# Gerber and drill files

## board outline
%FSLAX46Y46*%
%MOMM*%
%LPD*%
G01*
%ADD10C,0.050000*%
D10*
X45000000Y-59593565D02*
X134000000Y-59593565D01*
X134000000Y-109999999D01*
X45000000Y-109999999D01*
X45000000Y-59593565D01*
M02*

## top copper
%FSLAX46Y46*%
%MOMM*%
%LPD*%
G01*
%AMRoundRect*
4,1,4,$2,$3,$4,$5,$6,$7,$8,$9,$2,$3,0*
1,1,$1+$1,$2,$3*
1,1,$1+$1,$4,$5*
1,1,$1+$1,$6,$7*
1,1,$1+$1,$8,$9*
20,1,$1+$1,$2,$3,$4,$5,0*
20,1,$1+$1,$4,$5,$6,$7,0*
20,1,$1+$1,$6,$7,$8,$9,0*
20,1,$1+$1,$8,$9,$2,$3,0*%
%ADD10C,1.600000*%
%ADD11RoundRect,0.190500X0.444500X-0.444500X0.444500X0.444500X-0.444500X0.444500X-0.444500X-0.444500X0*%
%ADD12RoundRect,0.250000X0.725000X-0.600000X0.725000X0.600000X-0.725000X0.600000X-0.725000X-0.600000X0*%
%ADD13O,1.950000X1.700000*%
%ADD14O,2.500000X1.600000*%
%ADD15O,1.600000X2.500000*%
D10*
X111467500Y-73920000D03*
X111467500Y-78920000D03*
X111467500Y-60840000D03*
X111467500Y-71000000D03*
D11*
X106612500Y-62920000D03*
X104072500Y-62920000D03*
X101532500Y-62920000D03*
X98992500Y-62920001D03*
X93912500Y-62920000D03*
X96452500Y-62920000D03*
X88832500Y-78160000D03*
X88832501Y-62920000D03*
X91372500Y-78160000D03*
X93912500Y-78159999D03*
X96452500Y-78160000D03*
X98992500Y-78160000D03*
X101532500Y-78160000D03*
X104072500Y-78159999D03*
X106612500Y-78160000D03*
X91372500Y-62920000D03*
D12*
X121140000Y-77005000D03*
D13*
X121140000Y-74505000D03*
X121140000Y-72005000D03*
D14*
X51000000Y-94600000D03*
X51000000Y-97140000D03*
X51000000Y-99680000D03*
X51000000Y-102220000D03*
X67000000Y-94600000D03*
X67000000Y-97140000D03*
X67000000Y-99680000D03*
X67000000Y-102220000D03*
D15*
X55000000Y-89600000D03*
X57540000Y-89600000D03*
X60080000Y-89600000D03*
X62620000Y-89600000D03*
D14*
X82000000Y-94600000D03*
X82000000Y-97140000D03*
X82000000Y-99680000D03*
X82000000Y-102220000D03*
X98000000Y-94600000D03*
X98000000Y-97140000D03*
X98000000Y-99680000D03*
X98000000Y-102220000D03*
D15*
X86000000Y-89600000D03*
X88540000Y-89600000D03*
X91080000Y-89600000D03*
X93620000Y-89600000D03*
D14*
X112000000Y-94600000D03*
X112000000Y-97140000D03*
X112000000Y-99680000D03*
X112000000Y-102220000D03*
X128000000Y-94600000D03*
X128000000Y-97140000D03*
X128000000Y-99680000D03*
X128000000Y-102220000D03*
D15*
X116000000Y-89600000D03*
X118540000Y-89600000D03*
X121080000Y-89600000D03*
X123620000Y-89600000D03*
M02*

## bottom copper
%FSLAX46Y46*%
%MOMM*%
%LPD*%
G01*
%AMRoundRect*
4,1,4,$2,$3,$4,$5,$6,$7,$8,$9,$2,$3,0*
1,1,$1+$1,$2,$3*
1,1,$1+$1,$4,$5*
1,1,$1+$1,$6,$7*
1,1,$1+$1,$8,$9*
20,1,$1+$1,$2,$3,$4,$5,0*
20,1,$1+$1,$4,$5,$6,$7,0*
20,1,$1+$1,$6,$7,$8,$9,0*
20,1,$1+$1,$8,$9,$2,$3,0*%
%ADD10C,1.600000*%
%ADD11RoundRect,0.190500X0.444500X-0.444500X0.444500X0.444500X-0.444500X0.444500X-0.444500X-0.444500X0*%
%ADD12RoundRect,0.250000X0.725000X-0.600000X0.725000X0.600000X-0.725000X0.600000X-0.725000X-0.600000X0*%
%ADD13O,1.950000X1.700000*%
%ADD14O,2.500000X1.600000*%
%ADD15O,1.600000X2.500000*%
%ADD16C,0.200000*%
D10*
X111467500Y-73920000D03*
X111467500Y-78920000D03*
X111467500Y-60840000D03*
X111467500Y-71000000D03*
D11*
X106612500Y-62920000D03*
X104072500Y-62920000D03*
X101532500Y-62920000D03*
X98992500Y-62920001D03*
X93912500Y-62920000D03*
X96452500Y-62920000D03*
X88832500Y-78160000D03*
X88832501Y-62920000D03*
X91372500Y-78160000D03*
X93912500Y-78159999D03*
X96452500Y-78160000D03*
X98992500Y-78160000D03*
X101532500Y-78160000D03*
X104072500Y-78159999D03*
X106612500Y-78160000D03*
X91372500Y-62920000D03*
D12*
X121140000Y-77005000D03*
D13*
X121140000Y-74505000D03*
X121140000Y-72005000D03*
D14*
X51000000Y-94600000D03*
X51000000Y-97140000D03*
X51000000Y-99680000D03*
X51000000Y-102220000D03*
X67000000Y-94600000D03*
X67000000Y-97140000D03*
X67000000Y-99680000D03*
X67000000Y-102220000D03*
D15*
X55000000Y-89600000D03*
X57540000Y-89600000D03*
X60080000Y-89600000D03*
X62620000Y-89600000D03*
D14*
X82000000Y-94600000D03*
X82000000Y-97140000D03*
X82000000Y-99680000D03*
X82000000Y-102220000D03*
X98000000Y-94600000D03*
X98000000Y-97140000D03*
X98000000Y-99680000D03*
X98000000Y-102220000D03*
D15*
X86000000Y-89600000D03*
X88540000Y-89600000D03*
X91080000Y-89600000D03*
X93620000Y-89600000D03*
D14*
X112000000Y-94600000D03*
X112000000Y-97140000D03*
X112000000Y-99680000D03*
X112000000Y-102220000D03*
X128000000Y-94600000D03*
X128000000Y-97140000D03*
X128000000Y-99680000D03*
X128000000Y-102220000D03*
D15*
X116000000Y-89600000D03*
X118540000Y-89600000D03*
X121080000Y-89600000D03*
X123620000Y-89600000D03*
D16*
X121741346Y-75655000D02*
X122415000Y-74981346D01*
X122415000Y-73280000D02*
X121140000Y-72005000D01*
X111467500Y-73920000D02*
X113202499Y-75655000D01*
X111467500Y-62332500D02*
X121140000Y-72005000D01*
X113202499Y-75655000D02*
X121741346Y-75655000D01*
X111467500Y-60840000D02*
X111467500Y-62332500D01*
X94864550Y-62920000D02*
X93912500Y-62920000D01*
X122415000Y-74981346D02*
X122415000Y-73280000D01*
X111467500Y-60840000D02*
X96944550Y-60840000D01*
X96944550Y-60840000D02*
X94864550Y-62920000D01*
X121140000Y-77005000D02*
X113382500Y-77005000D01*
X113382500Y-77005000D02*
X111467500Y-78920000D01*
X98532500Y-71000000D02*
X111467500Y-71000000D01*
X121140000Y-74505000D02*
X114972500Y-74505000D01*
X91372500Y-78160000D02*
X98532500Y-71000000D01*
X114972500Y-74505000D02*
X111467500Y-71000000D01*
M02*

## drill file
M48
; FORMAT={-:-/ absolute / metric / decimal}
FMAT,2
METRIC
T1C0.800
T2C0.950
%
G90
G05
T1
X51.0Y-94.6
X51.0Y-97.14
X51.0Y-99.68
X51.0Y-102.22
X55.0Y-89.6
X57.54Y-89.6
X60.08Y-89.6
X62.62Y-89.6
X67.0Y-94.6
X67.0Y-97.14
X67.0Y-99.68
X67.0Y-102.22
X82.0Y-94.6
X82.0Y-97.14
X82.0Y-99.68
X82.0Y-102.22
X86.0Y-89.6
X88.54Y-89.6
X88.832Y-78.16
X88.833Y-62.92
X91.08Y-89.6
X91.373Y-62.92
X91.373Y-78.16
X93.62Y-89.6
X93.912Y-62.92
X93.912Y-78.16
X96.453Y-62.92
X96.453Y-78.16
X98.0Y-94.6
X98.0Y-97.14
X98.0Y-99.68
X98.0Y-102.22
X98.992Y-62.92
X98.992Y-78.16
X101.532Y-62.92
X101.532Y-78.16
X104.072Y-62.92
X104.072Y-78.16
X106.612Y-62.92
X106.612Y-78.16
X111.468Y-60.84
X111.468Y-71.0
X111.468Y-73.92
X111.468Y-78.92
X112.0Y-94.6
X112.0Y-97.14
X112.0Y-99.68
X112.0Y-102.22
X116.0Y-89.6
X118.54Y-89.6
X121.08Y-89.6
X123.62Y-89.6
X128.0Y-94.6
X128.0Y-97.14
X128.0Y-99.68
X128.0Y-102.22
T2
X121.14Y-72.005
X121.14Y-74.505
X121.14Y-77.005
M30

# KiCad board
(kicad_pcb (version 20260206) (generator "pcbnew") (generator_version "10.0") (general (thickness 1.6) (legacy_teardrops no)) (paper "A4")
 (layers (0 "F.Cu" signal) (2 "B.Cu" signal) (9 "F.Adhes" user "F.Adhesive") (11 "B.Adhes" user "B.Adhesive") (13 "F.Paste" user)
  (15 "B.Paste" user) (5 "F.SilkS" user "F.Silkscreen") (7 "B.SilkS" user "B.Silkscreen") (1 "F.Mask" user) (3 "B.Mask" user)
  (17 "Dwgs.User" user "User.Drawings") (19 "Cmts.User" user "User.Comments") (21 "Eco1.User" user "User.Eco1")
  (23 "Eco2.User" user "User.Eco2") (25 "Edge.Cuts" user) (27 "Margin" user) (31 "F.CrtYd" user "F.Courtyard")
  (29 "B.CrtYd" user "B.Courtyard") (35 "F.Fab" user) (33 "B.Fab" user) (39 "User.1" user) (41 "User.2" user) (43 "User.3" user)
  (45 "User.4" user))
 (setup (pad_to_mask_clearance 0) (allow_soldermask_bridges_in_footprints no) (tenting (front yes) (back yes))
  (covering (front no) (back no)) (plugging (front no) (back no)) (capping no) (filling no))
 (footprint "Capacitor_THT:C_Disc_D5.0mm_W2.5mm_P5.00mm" (layer "F.Cu") (at 111.4675 73.92 -90)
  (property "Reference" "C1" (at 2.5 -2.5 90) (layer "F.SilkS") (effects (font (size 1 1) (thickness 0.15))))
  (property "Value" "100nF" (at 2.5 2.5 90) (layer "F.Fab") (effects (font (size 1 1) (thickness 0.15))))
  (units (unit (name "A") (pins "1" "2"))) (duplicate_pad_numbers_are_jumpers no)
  (pad "1" thru_hole circle (at 0 0 270) (size 1.6 1.6) (drill 0.8) (layers "*.Cu" "*.Mask") (remove_unused_layers no) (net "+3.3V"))
  (pad "2" thru_hole circle (at 5 0 270) (size 1.6 1.6) (drill 0.8) (layers "*.Cu" "*.Mask") (remove_unused_layers no) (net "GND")))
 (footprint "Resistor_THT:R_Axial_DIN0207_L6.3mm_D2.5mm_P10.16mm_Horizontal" (layer "F.Cu") (at 111.4675 60.84 -90)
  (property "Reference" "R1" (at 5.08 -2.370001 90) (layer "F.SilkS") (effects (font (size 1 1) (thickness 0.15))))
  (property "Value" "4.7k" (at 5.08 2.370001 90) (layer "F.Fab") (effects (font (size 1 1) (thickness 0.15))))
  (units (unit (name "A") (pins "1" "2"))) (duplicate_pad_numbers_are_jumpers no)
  (pad "1" thru_hole circle (at 0 0 270) (size 1.6 1.6) (drill 0.8) (layers "*.Cu" "*.Mask") (remove_unused_layers no) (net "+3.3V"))
  (pad "2" thru_hole circle (at 10.16 0 270) (size 1.6 1.6) (drill 0.8) (layers "*.Cu" "*.Mask") (remove_unused_layers no)
   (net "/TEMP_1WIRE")))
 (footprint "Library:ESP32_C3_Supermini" (layer "F.Cu") (at 98.9925 68 90)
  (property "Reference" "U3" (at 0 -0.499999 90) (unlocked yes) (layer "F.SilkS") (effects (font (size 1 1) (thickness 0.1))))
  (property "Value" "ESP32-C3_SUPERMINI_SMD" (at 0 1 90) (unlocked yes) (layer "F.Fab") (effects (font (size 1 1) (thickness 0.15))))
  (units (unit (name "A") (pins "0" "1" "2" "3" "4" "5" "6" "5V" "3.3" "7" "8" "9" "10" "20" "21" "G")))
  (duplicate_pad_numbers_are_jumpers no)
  (pad "0" thru_hole roundrect (at 5.08 7.62 90) (size 1.27 1.27) (drill 0.8) (layers "*.Cu" "*.Mask") (remove_unused_layers no)
   (roundrect_rratio 0.15) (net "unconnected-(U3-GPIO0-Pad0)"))
  (pad "1" thru_hole roundrect (at 5.08 5.08 90) (size 1.27 1.27) (drill 0.8) (layers "*.Cu" "*.Mask") (remove_unused_layers no)
   (roundrect_rratio 0.15) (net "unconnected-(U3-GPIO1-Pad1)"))
  (pad "2" thru_hole roundrect (at 5.08 2.54 90) (size 1.27 1.27) (drill 0.8) (layers "*.Cu" "*.Mask") (remove_unused_layers no)
   (roundrect_rratio 0.15) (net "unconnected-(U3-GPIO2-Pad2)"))
  (pad "3" thru_hole roundrect (at 5.079999 0 90) (size 1.27 1.27) (drill 0.8) (layers "*.Cu" "*.Mask") (remove_unused_layers no)
   (roundrect_rratio 0.15) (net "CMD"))
  (pad "3.3" thru_hole roundrect (at 5.08 -5.08 90) (size 1.27 1.27) (drill 0.8) (layers "*.Cu" "*.Mask") (remove_unused_layers no)
   (roundrect_rratio 0.15) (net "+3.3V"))
  (pad "4" thru_hole roundrect (at 5.08 -2.54 90) (size 1.27 1.27) (drill 0.8) (layers "*.Cu" "*.Mask") (remove_unused_layers no)
   (roundrect_rratio 0.15) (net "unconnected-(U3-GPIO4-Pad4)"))
  (pad "5" thru_hole roundrect (at -10.16 -10.16 90) (size 1.27 1.27) (drill 0.8) (layers "*.Cu" "*.Mask") (remove_unused_layers no)
   (roundrect_rratio 0.15) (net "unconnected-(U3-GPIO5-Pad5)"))
  (pad "5V" thru_hole roundrect (at 5.08 -10.159999 90) (size 1.27 1.27) (drill 0.8) (layers "*.Cu" "*.Mask") (remove_unused_layers no)
   (roundrect_rratio 0.15) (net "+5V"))
  (pad "6" thru_hole roundrect (at -10.16 -7.62 90) (size 1.27 1.27) (drill 0.8) (layers "*.Cu" "*.Mask") (remove_unused_layers no)
   (roundrect_rratio 0.15) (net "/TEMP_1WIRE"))
  (pad "7" thru_hole roundrect (at -10.159999 -5.08 90) (size 1.27 1.27) (drill 0.8) (layers "*.Cu" "*.Mask") (remove_unused_layers no)
   (roundrect_rratio 0.15) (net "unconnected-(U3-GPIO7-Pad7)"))
  (pad "8" thru_hole roundrect (at -10.16 -2.54 90) (size 1.27 1.27) (drill 0.8) (layers "*.Cu" "*.Mask") (remove_unused_layers no)
   (roundrect_rratio 0.15) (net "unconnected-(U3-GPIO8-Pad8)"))
  (pad "9" thru_hole roundrect (at -10.16 0 90) (size 1.27 1.27) (drill 0.8) (layers "*.Cu" "*.Mask") (remove_unused_layers no)
   (roundrect_rratio 0.15) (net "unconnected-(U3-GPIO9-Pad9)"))
  (pad "10" thru_hole roundrect (at -10.16 2.54 90) (size 1.27 1.27) (drill 0.8) (layers "*.Cu" "*.Mask") (remove_unused_layers no)
   (roundrect_rratio 0.15) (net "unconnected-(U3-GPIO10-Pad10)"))
  (pad "20" thru_hole roundrect (at -10.159999 5.08 90) (size 1.27 1.27) (drill 0.8) (layers "*.Cu" "*.Mask") (remove_unused_layers no)
   (roundrect_rratio 0.15) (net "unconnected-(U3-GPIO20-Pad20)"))
  (pad "21" thru_hole roundrect (at -10.16 7.62 90) (size 1.27 1.27) (drill 0.8) (layers "*.Cu" "*.Mask") (remove_unused_layers no)
   (roundrect_rratio 0.15) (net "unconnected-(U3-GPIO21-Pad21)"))
  (pad "G" thru_hole roundrect (at 5.08 -7.62 90) (size 1.27 1.27) (drill 0.8) (layers "*.Cu" "*.Mask") (remove_unused_layers no)
   (roundrect_rratio 0.15) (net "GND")))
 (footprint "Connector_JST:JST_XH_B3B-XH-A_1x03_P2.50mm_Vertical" (layer "F.Cu") (at 121.14 77.005 90)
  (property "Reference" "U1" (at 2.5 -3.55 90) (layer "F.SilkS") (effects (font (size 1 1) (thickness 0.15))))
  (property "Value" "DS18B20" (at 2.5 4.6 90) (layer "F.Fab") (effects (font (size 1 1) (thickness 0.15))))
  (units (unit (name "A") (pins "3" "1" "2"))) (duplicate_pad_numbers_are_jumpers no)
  (pad "1" thru_hole roundrect (at 0 0 90) (size 1.7 1.95) (drill 0.95) (layers "*.Cu" "*.Mask") (remove_unused_layers no)
   (roundrect_rratio 0.147059) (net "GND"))
  (pad "2" thru_hole oval (at 2.5 0 90) (size 1.7 1.95) (drill 0.95) (layers "*.Cu" "*.Mask") (remove_unused_layers no) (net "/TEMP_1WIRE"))
  (pad "3" thru_hole oval (at 5 0 90) (size 1.7 1.95) (drill 0.95) (layers "*.Cu" "*.Mask") (remove_unused_layers no) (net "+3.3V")))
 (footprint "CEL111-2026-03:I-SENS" (layer "F.Cu") (at 59 87.1)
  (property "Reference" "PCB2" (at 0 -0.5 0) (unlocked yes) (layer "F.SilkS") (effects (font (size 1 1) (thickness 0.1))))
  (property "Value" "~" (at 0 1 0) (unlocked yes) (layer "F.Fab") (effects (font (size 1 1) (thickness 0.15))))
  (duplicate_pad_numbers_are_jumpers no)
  (pad "1" thru_hole oval (at -8 7.5 270) (size 1.6 2.5) (drill 0.8) (layers "*.Cu" "*.Mask") (remove_unused_layers no))
  (pad "2" thru_hole oval (at -8 10.04 270) (size 1.6 2.5) (drill 0.8) (layers "*.Cu" "*.Mask") (remove_unused_layers no))
  (pad "3" thru_hole oval (at -8 12.58 270) (size 1.6 2.5) (drill 0.8) (layers "*.Cu" "*.Mask") (remove_unused_layers no))
  (pad "4" thru_hole oval (at -8 15.12 270) (size 1.6 2.5) (drill 0.8) (layers "*.Cu" "*.Mask") (remove_unused_layers no))
  (pad "5" thru_hole oval (at 8 7.5 270) (size 1.6 2.5) (drill 0.8) (layers "*.Cu" "*.Mask") (remove_unused_layers no))
  (pad "6" thru_hole oval (at 8 10.04 270) (size 1.6 2.5) (drill 0.8) (layers "*.Cu" "*.Mask") (remove_unused_layers no))
  (pad "7" thru_hole oval (at 8 12.58 270) (size 1.6 2.5) (drill 0.8) (layers "*.Cu" "*.Mask") (remove_unused_layers no))
  (pad "8" thru_hole oval (at 8 15.12 270) (size 1.6 2.5) (drill 0.8) (layers "*.Cu" "*.Mask") (remove_unused_layers no))
  (pad "9" thru_hole oval (at -4 2.5) (size 1.6 2.5) (drill 0.8) (layers "*.Cu" "*.Mask") (remove_unused_layers no))
  (pad "10" thru_hole oval (at -1.46 2.5) (size 1.6 2.5) (drill 0.8) (layers "*.Cu" "*.Mask") (remove_unused_layers no))
  (pad "11" thru_hole oval (at 1.08 2.5) (size 1.6 2.5) (drill 0.8) (layers "*.Cu" "*.Mask") (remove_unused_layers no))
  (pad "12" thru_hole oval (at 3.62 2.5) (size 1.6 2.5) (drill 0.8) (layers "*.Cu" "*.Mask") (remove_unused_layers no)))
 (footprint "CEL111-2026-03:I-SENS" (layer "F.Cu") (at 90 87.1)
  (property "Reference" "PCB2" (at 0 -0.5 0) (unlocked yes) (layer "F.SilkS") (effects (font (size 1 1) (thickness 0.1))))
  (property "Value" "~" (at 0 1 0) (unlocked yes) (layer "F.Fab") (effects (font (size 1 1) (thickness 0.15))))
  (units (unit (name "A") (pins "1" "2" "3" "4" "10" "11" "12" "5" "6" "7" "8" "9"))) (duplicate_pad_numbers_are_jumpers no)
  (pad "1" thru_hole oval (at -8 7.5 270) (size 1.6 2.5) (drill 0.8) (layers "*.Cu" "*.Mask") (remove_unused_layers no) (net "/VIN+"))
  (pad "2" thru_hole oval (at -8 10.04 270) (size 1.6 2.5) (drill 0.8) (layers "*.Cu" "*.Mask") (remove_unused_layers no) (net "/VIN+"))
  (pad "3" thru_hole oval (at -8 12.58 270) (size 1.6 2.5) (drill 0.8) (layers "*.Cu" "*.Mask") (remove_unused_layers no) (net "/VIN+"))
  (pad "4" thru_hole oval (at -8 15.12 270) (size 1.6 2.5) (drill 0.8) (layers "*.Cu" "*.Mask") (remove_unused_layers no) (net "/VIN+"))
  (pad "5" thru_hole oval (at 8 7.5 270) (size 1.6 2.5) (drill 0.8) (layers "*.Cu" "*.Mask") (remove_unused_layers no)
   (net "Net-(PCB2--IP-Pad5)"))
  (pad "6" thru_hole oval (at 8 10.04 270) (size 1.6 2.5) (drill 0.8) (layers "*.Cu" "*.Mask") (remove_unused_layers no)
   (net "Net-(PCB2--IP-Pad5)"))
  (pad "7" thru_hole oval (at 8 12.58 270) (size 1.6 2.5) (drill 0.8) (layers "*.Cu" "*.Mask") (remove_unused_layers no)
   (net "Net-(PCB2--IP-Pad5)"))
  (pad "8" thru_hole oval (at 8 15.12 270) (size 1.6 2.5) (drill 0.8) (layers "*.Cu" "*.Mask") (remove_unused_layers no)
   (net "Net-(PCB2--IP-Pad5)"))
  (pad "9" thru_hole oval (at -4 2.5) (size 1.6 2.5) (drill 0.8) (layers "*.Cu" "*.Mask") (remove_unused_layers no) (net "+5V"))
  (pad "10" thru_hole oval (at -1.46 2.5) (size 1.6 2.5) (drill 0.8) (layers "*.Cu" "*.Mask") (remove_unused_layers no) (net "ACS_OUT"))
  (pad "11" thru_hole oval (at 1.08 2.5) (size 1.6 2.5) (drill 0.8) (layers "*.Cu" "*.Mask") (remove_unused_layers no) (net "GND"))
  (pad "12" thru_hole oval (at 3.62 2.5) (size 1.6 2.5) (drill 0.8) (layers "*.Cu" "*.Mask") (remove_unused_layers no) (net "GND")))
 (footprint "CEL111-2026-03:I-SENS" (layer "F.Cu") (at 120 87.1)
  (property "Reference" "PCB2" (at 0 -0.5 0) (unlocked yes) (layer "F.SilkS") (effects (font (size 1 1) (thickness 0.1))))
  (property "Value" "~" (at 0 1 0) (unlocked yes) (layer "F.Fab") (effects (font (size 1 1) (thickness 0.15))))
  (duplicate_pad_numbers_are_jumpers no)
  (pad "1" thru_hole oval (at -8 7.5 270) (size 1.6 2.5) (drill 0.8) (layers "*.Cu" "*.Mask") (remove_unused_layers no))
  (pad "2" thru_hole oval (at -8 10.04 270) (size 1.6 2.5) (drill 0.8) (layers "*.Cu" "*.Mask") (remove_unused_layers no))
  (pad "3" thru_hole oval (at -8 12.58 270) (size 1.6 2.5) (drill 0.8) (layers "*.Cu" "*.Mask") (remove_unused_layers no))
  (pad "4" thru_hole oval (at -8 15.12 270) (size 1.6 2.5) (drill 0.8) (layers "*.Cu" "*.Mask") (remove_unused_layers no))
  (pad "5" thru_hole oval (at 8 7.5 270) (size 1.6 2.5) (drill 0.8) (layers "*.Cu" "*.Mask") (remove_unused_layers no))
  (pad "6" thru_hole oval (at 8 10.04 270) (size 1.6 2.5) (drill 0.8) (layers "*.Cu" "*.Mask") (remove_unused_layers no))
  (pad "7" thru_hole oval (at 8 12.58 270) (size 1.6 2.5) (drill 0.8) (layers "*.Cu" "*.Mask") (remove_unused_layers no))
  (pad "8" thru_hole oval (at 8 15.12 270) (size 1.6 2.5) (drill 0.8) (layers "*.Cu" "*.Mask") (remove_unused_layers no))
  (pad "9" thru_hole oval (at -4 2.5) (size 1.6 2.5) (drill 0.8) (layers "*.Cu" "*.Mask") (remove_unused_layers no))
  (pad "10" thru_hole oval (at -1.46 2.5) (size 1.6 2.5) (drill 0.8) (layers "*.Cu" "*.Mask") (remove_unused_layers no))
  (pad "11" thru_hole oval (at 1.08 2.5) (size 1.6 2.5) (drill 0.8) (layers "*.Cu" "*.Mask") (remove_unused_layers no))
  (pad "12" thru_hole oval (at 3.62 2.5) (size 1.6 2.5) (drill 0.8) (layers "*.Cu" "*.Mask") (remove_unused_layers no)))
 (gr_rect (start 45 59.593565) (end 134 109.999999) (stroke (width 0.05) (type solid)) (fill no) (layer "Edge.Cuts"))
 (segment (start 121.741346 75.655) (end 122.415 74.981346) (width 0.2) (layer "B.Cu") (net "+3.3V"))
 (segment (start 122.415 73.28) (end 121.14 72.005) (width 0.2) (layer "B.Cu") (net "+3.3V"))
 (segment (start 111.4675 73.92) (end 113.202499 75.655) (width 0.2) (layer "B.Cu") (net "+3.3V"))
 (segment (start 111.4675 62.3325) (end 121.14 72.005) (width 0.2) (layer "B.Cu") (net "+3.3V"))
 (segment (start 113.202499 75.655) (end 121.741346 75.655) (width 0.2) (layer "B.Cu") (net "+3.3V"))
 (segment (start 111.4675 60.84) (end 111.4675 62.3325) (width 0.2) (layer "B.Cu") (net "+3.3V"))
 (segment (start 94.86455 62.92) (end 93.9125 62.92) (width 0.2) (layer "B.Cu") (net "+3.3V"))
 (segment (start 122.415 74.981346) (end 122.415 73.28) (width 0.2) (layer "B.Cu") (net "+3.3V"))
 (segment (start 111.4675 60.84) (end 96.94455 60.84) (width 0.2) (layer "B.Cu") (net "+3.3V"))
 (segment (start 96.94455 60.84) (end 94.86455 62.92) (width 0.2) (layer "B.Cu") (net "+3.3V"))
 (segment (start 121.14 77.005) (end 113.3825 77.005) (width 0.2) (layer "B.Cu") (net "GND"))
 (segment (start 113.3825 77.005) (end 111.4675 78.92) (width 0.2) (layer "B.Cu") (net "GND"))
 (segment (start 98.5325 71) (end 111.4675 71) (width 0.2) (layer "B.Cu") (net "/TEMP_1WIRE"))
 (segment (start 121.14 74.505) (end 114.9725 74.505) (width 0.2) (layer "B.Cu") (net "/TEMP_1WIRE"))
 (segment (start 91.3725 78.16) (end 98.5325 71) (width 0.2) (layer "B.Cu") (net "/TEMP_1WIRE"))
 (segment (start 114.9725 74.505) (end 111.4675 71) (width 0.2) (layer "B.Cu") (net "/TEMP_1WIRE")))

